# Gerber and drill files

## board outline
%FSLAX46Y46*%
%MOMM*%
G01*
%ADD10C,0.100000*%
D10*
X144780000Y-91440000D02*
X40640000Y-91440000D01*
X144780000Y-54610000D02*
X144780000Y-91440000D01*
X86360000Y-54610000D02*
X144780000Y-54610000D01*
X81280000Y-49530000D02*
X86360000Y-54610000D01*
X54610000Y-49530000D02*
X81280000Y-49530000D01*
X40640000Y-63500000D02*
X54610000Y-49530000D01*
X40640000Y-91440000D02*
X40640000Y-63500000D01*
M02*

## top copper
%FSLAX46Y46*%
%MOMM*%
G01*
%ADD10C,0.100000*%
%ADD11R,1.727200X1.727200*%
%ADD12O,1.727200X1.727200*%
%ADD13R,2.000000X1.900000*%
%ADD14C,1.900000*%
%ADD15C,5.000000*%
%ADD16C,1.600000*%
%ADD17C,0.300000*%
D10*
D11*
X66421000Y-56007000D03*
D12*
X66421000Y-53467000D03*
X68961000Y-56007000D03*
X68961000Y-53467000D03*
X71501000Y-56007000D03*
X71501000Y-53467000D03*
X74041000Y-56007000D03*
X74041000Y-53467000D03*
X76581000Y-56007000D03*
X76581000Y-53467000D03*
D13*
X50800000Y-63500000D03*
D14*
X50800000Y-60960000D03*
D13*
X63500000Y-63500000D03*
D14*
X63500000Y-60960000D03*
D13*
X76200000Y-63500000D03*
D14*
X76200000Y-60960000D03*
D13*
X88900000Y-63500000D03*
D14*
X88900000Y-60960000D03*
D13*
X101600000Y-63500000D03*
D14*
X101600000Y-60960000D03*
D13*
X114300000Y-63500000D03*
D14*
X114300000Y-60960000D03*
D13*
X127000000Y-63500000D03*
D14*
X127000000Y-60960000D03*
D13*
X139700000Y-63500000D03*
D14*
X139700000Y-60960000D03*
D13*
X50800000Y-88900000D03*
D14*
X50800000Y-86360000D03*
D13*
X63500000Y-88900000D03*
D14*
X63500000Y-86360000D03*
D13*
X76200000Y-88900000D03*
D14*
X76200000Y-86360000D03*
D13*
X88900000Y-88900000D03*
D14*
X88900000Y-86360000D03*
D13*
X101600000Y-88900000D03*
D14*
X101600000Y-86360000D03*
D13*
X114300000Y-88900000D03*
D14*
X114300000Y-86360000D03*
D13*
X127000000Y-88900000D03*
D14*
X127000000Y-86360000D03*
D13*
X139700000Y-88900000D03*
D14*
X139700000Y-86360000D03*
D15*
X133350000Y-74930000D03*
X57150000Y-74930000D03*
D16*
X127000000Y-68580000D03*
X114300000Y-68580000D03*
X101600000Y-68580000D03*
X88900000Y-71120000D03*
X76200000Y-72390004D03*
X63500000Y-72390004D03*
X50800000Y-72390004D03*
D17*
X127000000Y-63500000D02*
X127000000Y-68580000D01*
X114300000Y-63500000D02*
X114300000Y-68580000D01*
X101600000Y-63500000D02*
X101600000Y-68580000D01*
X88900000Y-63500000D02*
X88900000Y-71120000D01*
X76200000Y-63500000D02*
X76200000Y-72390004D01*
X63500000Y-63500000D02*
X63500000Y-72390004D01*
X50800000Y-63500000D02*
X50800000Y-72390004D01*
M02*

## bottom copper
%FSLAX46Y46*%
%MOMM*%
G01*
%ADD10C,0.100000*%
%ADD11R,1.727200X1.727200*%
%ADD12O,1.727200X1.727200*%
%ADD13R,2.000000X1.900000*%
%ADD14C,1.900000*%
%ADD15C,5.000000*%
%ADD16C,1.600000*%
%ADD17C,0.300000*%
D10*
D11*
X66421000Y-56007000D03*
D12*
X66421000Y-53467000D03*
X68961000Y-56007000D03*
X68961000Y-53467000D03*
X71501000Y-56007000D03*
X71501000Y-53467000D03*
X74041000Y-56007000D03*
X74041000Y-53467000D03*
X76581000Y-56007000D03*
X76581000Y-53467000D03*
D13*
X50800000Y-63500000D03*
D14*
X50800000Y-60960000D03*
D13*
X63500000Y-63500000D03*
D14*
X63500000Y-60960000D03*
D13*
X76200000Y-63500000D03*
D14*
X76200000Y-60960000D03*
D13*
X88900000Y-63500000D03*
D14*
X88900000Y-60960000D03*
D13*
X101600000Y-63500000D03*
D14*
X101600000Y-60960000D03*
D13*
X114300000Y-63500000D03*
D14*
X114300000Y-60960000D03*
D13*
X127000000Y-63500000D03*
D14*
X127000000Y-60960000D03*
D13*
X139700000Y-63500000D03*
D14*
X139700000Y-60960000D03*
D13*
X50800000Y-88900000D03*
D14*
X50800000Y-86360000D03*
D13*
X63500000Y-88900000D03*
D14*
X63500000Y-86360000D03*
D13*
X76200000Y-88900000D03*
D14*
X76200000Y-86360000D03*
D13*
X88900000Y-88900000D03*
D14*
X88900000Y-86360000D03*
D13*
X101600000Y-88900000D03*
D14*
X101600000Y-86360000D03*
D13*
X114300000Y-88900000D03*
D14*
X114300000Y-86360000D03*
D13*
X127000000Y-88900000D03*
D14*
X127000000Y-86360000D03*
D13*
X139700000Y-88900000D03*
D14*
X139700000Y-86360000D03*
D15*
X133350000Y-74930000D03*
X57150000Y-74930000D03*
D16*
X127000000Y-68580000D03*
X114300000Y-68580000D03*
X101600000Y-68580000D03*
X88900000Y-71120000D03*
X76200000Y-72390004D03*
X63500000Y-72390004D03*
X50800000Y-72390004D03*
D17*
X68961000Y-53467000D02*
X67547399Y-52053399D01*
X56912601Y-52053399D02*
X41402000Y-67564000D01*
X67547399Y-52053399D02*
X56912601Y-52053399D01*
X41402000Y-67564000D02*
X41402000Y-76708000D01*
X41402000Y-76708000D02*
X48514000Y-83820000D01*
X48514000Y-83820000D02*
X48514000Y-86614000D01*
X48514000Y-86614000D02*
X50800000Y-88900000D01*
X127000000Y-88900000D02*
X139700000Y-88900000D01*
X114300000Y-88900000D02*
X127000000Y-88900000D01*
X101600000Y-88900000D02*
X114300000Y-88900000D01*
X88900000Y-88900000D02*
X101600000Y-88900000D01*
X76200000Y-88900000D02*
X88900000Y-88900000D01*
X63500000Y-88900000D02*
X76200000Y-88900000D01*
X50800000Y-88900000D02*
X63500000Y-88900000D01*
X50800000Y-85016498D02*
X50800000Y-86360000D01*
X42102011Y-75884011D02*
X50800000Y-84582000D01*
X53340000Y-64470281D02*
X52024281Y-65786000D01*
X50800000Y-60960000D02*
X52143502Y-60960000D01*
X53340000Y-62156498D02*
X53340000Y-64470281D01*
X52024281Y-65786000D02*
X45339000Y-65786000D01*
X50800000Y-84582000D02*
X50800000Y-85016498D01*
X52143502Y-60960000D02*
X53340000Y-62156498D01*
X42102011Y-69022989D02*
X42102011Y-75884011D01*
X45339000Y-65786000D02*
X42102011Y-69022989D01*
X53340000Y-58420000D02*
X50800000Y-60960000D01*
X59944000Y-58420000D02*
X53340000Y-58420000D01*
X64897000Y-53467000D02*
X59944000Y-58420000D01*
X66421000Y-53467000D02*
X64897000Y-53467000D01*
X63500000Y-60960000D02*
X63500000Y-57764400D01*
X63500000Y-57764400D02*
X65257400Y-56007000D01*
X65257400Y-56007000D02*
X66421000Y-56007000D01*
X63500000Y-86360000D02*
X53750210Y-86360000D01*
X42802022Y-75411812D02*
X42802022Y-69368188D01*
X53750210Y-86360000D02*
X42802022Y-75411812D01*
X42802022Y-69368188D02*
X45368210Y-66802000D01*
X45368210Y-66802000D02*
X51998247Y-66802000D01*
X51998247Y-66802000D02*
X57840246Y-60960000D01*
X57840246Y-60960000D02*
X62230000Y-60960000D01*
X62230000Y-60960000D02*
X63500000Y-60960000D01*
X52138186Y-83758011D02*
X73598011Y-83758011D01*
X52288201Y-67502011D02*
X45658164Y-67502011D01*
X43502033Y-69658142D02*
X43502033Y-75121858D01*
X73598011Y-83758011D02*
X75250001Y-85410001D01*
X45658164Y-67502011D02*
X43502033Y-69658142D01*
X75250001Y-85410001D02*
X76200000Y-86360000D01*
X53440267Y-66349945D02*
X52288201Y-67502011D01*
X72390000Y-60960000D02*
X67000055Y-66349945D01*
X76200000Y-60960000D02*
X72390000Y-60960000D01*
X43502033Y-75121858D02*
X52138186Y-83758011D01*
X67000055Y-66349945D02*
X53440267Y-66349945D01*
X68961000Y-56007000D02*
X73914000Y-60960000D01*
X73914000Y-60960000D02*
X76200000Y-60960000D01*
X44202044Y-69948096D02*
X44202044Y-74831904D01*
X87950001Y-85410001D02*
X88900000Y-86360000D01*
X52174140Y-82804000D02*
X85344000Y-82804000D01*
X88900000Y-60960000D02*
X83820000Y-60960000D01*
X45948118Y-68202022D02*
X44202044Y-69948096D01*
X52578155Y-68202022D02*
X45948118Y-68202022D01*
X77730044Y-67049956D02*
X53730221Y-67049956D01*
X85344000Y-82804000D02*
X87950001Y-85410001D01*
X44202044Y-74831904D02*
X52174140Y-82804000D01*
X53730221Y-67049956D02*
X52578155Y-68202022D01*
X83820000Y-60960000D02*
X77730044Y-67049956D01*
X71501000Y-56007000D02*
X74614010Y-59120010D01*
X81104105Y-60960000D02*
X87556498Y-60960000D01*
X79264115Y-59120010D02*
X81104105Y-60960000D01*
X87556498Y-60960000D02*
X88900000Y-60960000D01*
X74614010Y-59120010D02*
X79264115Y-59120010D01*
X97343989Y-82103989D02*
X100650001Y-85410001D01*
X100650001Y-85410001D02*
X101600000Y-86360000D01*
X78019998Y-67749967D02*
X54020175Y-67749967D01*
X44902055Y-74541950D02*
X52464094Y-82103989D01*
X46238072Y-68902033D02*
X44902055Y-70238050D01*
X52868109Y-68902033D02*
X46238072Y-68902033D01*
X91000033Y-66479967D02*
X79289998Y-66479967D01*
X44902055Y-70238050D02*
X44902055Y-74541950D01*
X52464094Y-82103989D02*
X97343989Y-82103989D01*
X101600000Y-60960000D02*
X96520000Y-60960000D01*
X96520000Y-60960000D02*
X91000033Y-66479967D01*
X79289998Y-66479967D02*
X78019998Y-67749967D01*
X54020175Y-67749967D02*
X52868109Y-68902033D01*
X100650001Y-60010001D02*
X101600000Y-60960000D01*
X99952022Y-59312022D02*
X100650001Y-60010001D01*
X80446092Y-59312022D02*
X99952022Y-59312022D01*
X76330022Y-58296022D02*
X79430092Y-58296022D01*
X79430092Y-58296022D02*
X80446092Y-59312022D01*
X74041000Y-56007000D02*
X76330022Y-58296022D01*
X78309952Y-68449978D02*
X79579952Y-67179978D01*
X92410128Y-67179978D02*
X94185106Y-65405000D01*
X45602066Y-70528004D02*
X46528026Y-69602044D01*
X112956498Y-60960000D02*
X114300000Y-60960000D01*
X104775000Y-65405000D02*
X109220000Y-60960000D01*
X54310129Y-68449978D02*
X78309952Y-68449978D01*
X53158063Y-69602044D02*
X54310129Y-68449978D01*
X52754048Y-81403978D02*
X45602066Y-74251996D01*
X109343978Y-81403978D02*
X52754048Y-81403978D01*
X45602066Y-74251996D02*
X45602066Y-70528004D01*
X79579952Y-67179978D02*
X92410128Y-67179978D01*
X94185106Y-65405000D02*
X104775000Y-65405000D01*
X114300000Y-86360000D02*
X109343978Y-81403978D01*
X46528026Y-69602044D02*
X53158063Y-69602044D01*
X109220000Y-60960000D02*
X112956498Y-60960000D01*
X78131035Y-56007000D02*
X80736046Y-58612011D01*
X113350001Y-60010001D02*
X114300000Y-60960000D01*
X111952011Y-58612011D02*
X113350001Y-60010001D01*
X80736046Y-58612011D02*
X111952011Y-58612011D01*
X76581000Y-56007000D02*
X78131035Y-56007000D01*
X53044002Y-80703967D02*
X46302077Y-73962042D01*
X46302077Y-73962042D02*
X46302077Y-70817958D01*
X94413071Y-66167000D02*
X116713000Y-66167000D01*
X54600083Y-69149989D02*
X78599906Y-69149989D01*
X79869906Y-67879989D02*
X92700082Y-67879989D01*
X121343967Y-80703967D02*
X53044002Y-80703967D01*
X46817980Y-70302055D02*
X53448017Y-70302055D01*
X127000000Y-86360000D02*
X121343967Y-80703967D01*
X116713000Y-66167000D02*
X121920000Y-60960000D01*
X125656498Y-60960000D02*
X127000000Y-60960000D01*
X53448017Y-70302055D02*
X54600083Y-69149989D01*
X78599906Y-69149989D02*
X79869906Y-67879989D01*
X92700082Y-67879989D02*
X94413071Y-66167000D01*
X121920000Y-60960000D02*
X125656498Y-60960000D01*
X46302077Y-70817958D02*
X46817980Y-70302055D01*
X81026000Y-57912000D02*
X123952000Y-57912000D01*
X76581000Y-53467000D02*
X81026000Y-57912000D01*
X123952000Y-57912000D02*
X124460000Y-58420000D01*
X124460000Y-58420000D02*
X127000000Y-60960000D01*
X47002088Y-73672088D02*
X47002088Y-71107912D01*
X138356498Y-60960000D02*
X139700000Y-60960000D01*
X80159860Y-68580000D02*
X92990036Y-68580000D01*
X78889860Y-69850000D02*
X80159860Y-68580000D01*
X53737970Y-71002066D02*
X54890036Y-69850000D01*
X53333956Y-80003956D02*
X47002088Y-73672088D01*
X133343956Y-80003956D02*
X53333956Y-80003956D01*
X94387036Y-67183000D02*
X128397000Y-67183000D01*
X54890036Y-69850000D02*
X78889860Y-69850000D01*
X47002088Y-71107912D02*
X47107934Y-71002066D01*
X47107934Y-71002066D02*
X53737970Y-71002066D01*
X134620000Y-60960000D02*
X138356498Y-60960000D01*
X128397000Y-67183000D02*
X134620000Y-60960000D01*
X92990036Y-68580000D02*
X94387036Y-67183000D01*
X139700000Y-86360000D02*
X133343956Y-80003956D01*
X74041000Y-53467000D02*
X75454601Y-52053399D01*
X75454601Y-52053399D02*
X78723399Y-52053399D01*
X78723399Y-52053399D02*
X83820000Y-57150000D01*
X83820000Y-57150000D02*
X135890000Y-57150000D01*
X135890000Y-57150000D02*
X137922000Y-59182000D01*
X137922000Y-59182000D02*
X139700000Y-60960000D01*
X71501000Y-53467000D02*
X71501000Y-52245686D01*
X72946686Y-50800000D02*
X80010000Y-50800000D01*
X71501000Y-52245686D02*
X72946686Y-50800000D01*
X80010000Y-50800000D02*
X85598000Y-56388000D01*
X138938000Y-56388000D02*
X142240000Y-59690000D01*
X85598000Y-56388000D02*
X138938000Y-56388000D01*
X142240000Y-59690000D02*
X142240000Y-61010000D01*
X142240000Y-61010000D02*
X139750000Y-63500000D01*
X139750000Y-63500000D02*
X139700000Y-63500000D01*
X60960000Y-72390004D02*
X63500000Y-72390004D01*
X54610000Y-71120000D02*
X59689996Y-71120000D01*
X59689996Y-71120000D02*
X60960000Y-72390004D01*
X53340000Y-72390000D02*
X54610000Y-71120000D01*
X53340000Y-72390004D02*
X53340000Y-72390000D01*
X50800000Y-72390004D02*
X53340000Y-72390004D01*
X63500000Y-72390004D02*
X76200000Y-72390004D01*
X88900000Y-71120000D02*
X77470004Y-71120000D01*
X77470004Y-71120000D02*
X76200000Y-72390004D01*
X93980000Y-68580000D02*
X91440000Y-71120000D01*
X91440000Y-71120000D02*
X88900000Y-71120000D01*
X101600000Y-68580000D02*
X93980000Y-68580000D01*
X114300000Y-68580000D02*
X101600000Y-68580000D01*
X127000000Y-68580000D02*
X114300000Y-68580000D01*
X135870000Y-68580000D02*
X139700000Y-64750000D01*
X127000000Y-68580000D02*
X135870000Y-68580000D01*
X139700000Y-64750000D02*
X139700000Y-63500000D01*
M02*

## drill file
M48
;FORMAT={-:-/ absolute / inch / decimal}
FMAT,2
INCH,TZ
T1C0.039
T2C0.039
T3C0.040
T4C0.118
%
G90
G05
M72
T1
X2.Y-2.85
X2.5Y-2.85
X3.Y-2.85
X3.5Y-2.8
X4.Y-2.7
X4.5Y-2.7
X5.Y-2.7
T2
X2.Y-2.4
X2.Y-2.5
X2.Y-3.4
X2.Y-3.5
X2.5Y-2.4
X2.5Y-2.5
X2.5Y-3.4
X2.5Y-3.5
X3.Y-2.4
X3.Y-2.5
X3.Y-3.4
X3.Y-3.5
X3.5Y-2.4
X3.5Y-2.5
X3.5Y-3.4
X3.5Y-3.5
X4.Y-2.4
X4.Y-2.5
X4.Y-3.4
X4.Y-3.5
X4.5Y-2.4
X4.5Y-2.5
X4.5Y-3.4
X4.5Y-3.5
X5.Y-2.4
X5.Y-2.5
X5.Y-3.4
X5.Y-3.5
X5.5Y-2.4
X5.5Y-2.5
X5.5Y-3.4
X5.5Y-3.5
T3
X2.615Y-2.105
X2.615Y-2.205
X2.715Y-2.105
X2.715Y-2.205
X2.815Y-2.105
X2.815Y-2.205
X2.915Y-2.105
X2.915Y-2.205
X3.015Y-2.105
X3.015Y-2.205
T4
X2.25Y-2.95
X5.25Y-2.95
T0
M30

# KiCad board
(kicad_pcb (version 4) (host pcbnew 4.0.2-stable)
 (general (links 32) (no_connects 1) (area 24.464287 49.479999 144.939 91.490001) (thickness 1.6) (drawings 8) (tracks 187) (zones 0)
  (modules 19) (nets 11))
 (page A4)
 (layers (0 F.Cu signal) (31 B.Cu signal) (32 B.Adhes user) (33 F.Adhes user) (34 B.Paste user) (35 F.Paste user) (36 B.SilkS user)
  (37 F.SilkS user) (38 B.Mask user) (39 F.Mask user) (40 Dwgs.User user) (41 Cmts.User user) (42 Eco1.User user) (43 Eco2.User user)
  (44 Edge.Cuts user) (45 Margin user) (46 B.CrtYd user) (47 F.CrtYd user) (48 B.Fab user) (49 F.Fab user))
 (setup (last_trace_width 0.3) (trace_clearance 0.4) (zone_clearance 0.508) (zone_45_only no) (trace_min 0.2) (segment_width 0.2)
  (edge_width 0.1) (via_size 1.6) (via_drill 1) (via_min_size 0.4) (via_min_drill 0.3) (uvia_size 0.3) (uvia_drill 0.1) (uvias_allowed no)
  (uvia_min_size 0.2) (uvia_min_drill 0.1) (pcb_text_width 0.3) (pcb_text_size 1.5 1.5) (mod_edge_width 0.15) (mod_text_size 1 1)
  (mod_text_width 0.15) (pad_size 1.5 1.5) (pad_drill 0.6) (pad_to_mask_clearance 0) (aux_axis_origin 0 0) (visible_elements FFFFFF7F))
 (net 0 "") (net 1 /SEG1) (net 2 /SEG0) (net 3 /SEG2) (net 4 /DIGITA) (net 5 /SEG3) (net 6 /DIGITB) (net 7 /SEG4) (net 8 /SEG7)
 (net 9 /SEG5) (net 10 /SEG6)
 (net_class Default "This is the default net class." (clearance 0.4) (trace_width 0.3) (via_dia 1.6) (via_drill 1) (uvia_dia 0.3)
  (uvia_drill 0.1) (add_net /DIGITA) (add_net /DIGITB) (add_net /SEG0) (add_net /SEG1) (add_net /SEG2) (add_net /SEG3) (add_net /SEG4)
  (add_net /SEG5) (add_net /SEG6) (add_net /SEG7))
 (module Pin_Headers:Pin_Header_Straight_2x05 (layer F.Cu) (at 66.421 56.007 90)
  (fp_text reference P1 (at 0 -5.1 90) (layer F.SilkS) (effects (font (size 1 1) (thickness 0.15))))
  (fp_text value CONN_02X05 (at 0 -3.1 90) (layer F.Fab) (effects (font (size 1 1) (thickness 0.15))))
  (pad 1 thru_hole rect (at 0 0 90) (size 1.7272 1.7272) (drill 1.016) (layers *.Cu *.Mask F.SilkS) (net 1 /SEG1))
  (pad 2 thru_hole oval (at 2.54 0 90) (size 1.7272 1.7272) (drill 1.016) (layers *.Cu *.Mask F.SilkS) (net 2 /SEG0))
  (pad 3 thru_hole oval (at 0 2.54 90) (size 1.7272 1.7272) (drill 1.016) (layers *.Cu *.Mask F.SilkS) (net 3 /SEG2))
  (pad 4 thru_hole oval (at 2.54 2.54 90) (size 1.7272 1.7272) (drill 1.016) (layers *.Cu *.Mask F.SilkS) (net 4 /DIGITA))
  (pad 5 thru_hole oval (at 0 5.08 90) (size 1.7272 1.7272) (drill 1.016) (layers *.Cu *.Mask F.SilkS) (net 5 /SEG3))
  (pad 6 thru_hole oval (at 2.54 5.08 90) (size 1.7272 1.7272) (drill 1.016) (layers *.Cu *.Mask F.SilkS) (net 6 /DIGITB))
  (pad 7 thru_hole oval (at 0 7.62 90) (size 1.7272 1.7272) (drill 1.016) (layers *.Cu *.Mask F.SilkS) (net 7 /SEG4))
  (pad 8 thru_hole oval (at 2.54 7.62 90) (size 1.7272 1.7272) (drill 1.016) (layers *.Cu *.Mask F.SilkS) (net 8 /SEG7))
  (pad 9 thru_hole oval (at 0 10.16 90) (size 1.7272 1.7272) (drill 1.016) (layers *.Cu *.Mask F.SilkS) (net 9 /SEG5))
  (pad 10 thru_hole oval (at 2.54 10.16 90) (size 1.7272 1.7272) (drill 1.016) (layers *.Cu *.Mask F.SilkS) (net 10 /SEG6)))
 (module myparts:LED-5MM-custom (layer F.Cu) (at 50.8 63.5 90)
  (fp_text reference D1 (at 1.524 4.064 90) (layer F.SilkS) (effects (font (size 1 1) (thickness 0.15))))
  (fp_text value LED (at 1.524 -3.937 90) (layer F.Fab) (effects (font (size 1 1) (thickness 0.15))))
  (pad 1 thru_hole rect (at 0 0 180) (size 2 1.9) (drill 1.00076) (layers *.Cu *.Mask F.SilkS) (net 6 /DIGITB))
  (pad 2 thru_hole circle (at 2.54 0 90) (size 1.9 1.9) (drill 1.00076) (layers *.Cu *.Mask F.SilkS) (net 2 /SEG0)))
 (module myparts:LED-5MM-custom (layer F.Cu) (at 63.5 63.5 90)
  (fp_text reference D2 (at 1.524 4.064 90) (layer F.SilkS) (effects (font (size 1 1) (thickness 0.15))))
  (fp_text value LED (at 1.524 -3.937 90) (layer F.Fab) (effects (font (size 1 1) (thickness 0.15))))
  (pad 1 thru_hole rect (at 0 0 180) (size 2 1.9) (drill 1.00076) (layers *.Cu *.Mask F.SilkS) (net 6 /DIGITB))
  (pad 2 thru_hole circle (at 2.54 0 90) (size 1.9 1.9) (drill 1.00076) (layers *.Cu *.Mask F.SilkS) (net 1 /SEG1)))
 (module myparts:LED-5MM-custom (layer F.Cu) (at 76.2 63.5 90)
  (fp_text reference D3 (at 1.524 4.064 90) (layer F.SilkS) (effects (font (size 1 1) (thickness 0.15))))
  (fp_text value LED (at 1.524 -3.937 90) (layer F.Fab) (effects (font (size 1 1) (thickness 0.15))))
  (pad 1 thru_hole rect (at 0 0 180) (size 2 1.9) (drill 1.00076) (layers *.Cu *.Mask F.SilkS) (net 6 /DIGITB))
  (pad 2 thru_hole circle (at 2.54 0 90) (size 1.9 1.9) (drill 1.00076) (layers *.Cu *.Mask F.SilkS) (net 3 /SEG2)))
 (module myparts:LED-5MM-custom (layer F.Cu) (at 88.9 63.5 90)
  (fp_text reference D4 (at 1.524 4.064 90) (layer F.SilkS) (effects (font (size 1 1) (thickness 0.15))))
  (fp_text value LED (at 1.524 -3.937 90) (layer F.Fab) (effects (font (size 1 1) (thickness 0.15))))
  (pad 1 thru_hole rect (at 0 0 180) (size 2 1.9) (drill 1.00076) (layers *.Cu *.Mask F.SilkS) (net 6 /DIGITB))
  (pad 2 thru_hole circle (at 2.54 0 90) (size 1.9 1.9) (drill 1.00076) (layers *.Cu *.Mask F.SilkS) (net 5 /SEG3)))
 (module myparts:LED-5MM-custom (layer F.Cu) (at 101.6 63.5 90)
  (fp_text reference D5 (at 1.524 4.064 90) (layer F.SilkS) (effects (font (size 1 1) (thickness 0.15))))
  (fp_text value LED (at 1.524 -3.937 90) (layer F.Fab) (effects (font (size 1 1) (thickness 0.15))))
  (pad 1 thru_hole rect (at 0 0 180) (size 2 1.9) (drill 1.00076) (layers *.Cu *.Mask F.SilkS) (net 6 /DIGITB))
  (pad 2 thru_hole circle (at 2.54 0 90) (size 1.9 1.9) (drill 1.00076) (layers *.Cu *.Mask F.SilkS) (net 7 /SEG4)))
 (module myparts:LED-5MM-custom (layer F.Cu) (at 114.3 63.5 90)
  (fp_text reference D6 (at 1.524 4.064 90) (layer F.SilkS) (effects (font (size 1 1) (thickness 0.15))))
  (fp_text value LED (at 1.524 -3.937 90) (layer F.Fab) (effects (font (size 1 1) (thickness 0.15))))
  (pad 1 thru_hole rect (at 0 0 180) (size 2 1.9) (drill 1.00076) (layers *.Cu *.Mask F.SilkS) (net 6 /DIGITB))
  (pad 2 thru_hole circle (at 2.54 0 90) (size 1.9 1.9) (drill 1.00076) (layers *.Cu *.Mask F.SilkS) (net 9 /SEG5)))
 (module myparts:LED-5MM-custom (layer F.Cu) (at 127 63.5 90)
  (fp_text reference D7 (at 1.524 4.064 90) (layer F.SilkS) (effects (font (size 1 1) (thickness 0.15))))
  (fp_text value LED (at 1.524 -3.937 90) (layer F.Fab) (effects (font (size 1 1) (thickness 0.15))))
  (pad 1 thru_hole rect (at 0 0 180) (size 2 1.9) (drill 1.00076) (layers *.Cu *.Mask F.SilkS) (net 6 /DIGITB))
  (pad 2 thru_hole circle (at 2.54 0 90) (size 1.9 1.9) (drill 1.00076) (layers *.Cu *.Mask F.SilkS) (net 10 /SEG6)))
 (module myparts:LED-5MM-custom (layer F.Cu) (at 139.7 63.5 90)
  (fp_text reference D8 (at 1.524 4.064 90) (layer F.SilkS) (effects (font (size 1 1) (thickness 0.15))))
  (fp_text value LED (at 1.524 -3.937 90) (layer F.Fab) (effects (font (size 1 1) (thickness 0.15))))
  (pad 1 thru_hole rect (at 0 0 180) (size 2 1.9) (drill 1.00076) (layers *.Cu *.Mask F.SilkS) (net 6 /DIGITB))
  (pad 2 thru_hole circle (at 2.54 0 90) (size 1.9 1.9) (drill 1.00076) (layers *.Cu *.Mask F.SilkS) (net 8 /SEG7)))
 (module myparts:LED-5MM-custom (layer F.Cu) (at 50.8 88.9 90)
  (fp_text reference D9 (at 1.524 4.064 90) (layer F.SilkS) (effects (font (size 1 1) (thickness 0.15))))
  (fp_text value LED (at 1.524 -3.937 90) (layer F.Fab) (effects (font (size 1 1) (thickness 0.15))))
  (pad 1 thru_hole rect (at 0 0 180) (size 2 1.9) (drill 1.00076) (layers *.Cu *.Mask F.SilkS) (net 4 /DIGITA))
  (pad 2 thru_hole circle (at 2.54 0 90) (size 1.9 1.9) (drill 1.00076) (layers *.Cu *.Mask F.SilkS) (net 2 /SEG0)))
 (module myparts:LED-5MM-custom (layer F.Cu) (at 63.5 88.9 90)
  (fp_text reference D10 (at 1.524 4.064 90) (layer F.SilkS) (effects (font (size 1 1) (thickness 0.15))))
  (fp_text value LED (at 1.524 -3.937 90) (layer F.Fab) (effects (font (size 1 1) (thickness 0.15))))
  (pad 1 thru_hole rect (at 0 0 180) (size 2 1.9) (drill 1.00076) (layers *.Cu *.Mask F.SilkS) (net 4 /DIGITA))
  (pad 2 thru_hole circle (at 2.54 0 90) (size 1.9 1.9) (drill 1.00076) (layers *.Cu *.Mask F.SilkS) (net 1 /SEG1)))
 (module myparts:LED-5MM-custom (layer F.Cu) (at 76.2 88.9 90)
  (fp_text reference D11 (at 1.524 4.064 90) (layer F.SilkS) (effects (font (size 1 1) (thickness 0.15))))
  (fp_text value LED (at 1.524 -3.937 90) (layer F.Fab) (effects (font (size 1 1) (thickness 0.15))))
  (pad 1 thru_hole rect (at 0 0 180) (size 2 1.9) (drill 1.00076) (layers *.Cu *.Mask F.SilkS) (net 4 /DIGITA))
  (pad 2 thru_hole circle (at 2.54 0 90) (size 1.9 1.9) (drill 1.00076) (layers *.Cu *.Mask F.SilkS) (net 3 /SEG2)))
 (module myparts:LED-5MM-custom (layer F.Cu) (at 88.9 88.9 90)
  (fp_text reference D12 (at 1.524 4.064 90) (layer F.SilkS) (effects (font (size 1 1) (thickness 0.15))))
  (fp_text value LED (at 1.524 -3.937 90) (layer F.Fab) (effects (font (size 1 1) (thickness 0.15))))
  (pad 1 thru_hole rect (at 0 0 180) (size 2 1.9) (drill 1.00076) (layers *.Cu *.Mask F.SilkS) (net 4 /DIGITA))
  (pad 2 thru_hole circle (at 2.54 0 90) (size 1.9 1.9) (drill 1.00076) (layers *.Cu *.Mask F.SilkS) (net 5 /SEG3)))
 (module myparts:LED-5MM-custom (layer F.Cu) (at 101.6 88.9 90)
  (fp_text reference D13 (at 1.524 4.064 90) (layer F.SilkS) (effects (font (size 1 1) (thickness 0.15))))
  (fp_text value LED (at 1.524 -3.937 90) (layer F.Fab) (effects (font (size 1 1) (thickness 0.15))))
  (pad 1 thru_hole rect (at 0 0 180) (size 2 1.9) (drill 1.00076) (layers *.Cu *.Mask F.SilkS) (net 4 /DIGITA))
  (pad 2 thru_hole circle (at 2.54 0 90) (size 1.9 1.9) (drill 1.00076) (layers *.Cu *.Mask F.SilkS) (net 7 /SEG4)))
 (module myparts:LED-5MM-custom (layer F.Cu) (at 114.3 88.9 90)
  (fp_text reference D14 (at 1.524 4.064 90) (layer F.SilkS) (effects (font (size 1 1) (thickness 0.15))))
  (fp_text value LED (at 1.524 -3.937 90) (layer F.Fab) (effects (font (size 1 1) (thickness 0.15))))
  (pad 1 thru_hole rect (at 0 0 180) (size 2 1.9) (drill 1.00076) (layers *.Cu *.Mask F.SilkS) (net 4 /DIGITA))
  (pad 2 thru_hole circle (at 2.54 0 90) (size 1.9 1.9) (drill 1.00076) (layers *.Cu *.Mask F.SilkS) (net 9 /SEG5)))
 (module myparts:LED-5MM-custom (layer F.Cu) (at 127 88.9 90)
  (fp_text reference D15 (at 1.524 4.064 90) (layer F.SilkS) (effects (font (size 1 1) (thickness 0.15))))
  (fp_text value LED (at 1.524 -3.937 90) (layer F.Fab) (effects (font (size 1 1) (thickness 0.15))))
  (pad 1 thru_hole rect (at 0 0 180) (size 2 1.9) (drill 1.00076) (layers *.Cu *.Mask F.SilkS) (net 4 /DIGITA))
  (pad 2 thru_hole circle (at 2.54 0 90) (size 1.9 1.9) (drill 1.00076) (layers *.Cu *.Mask F.SilkS) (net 10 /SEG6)))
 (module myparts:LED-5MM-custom (layer F.Cu) (at 139.7 88.9 90)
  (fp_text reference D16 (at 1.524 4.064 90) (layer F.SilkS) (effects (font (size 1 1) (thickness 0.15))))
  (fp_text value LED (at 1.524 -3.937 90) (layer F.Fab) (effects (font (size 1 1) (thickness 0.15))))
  (pad 1 thru_hole rect (at 0 0 180) (size 2 1.9) (drill 1.00076) (layers *.Cu *.Mask F.SilkS) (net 4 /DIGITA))
  (pad 2 thru_hole circle (at 2.54 0 90) (size 1.9 1.9) (drill 1.00076) (layers *.Cu *.Mask F.SilkS) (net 8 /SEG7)))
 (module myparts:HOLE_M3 (layer F.Cu) (at 133.35 74.93)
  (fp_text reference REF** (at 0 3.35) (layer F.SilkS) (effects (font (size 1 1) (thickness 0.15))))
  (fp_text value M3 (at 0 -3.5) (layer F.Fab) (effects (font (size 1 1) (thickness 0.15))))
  (pad 1 thru_hole circle (at 0 0) (size 5 5) (drill 3) (layers *.Cu *.Mask F.SilkS)))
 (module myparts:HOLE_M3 (layer F.Cu) (at 57.15 74.93)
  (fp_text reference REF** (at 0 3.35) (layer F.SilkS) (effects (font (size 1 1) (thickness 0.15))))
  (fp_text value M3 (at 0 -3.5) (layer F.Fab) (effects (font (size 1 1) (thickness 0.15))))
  (pad 1 thru_hole circle (at 0 0) (size 5 5) (drill 3) (layers *.Cu *.Mask F.SilkS)))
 (gr_line (start 144.78 91.44) (end 40.64 91.44) (layer Edge.Cuts) (width 0.1))
 (gr_line (start 144.78 54.61) (end 144.78 91.44) (layer Edge.Cuts) (width 0.1))
 (gr_line (start 86.36 54.61) (end 144.78 54.61) (layer Edge.Cuts) (width 0.1))
 (gr_line (start 81.28 49.53) (end 86.36 54.61) (layer Edge.Cuts) (width 0.1))
 (gr_line (start 54.61 49.53) (end 81.28 49.53) (layer Edge.Cuts) (width 0.1))
 (gr_line (start 40.64 63.5) (end 54.61 49.53) (layer Edge.Cuts) (width 0.1))
 (gr_line (start 40.64 91.44) (end 40.64 63.5) (layer Edge.Cuts) (width 0.1))
 (segment (start 68.961 53.467) (end 67.547399 52.053399) (width 0.3) (layer B.Cu) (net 4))
 (segment (start 56.912601 52.053399) (end 41.402 67.564) (width 0.3) (layer B.Cu) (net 4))
 (segment (start 67.547399 52.053399) (end 56.912601 52.053399) (width 0.3) (layer B.Cu) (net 4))
 (segment (start 41.402 67.564) (end 41.402 76.708) (width 0.3) (layer B.Cu) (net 4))
 (segment (start 41.402 76.708) (end 48.514 83.82) (width 0.3) (layer B.Cu) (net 4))
 (segment (start 48.514 83.82) (end 48.514 86.614) (width 0.3) (layer B.Cu) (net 4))
 (segment (start 48.514 86.614) (end 50.8 88.9) (width 0.3) (layer B.Cu) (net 4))
 (segment (start 127 88.9) (end 139.7 88.9) (width 0.3) (layer B.Cu) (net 4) (status 30))
 (segment (start 114.3 88.9) (end 127 88.9) (width 0.3) (layer B.Cu) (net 4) (status 30))
 (segment (start 101.6 88.9) (end 114.3 88.9) (width 0.3) (layer B.Cu) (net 4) (status 30))
 (segment (start 88.9 88.9) (end 101.6 88.9) (width 0.3) (layer B.Cu) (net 4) (status 30))
 (segment (start 76.2 88.9) (end 88.9 88.9) (width 0.3) (layer B.Cu) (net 4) (status 30))
 (segment (start 63.5 88.9) (end 76.2 88.9) (width 0.3) (layer B.Cu) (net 4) (status 30))
 (segment (start 50.8 88.9) (end 63.5 88.9) (width 0.3) (layer B.Cu) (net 4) (status 30))
 (segment (start 50.8 85.016498) (end 50.8 86.36) (width 0.3) (layer B.Cu) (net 2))
 (segment (start 42.102011 75.884011) (end 50.8 84.582) (width 0.3) (layer B.Cu) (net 2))
 (segment (start 53.34 64.470281) (end 52.024281 65.786) (width 0.3) (layer B.Cu) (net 2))
 (segment (start 50.8 60.96) (end 52.143502 60.96) (width 0.3) (layer B.Cu) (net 2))
 (segment (start 53.34 62.156498) (end 53.34 64.470281) (width 0.3) (layer B.Cu) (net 2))
 (segment (start 52.024281 65.786) (end 45.339 65.786) (width 0.3) (layer B.Cu) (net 2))
 (segment (start 50.8 84.582) (end 50.8 85.016498) (width 0.3) (layer B.Cu) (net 2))
 (segment (start 52.143502 60.96) (end 53.34 62.156498) (width 0.3) (layer B.Cu) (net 2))
 (segment (start 42.102011 69.022989) (end 42.102011 75.884011) (width 0.3) (layer B.Cu) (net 2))
 (segment (start 45.339 65.786) (end 42.102011 69.022989) (width 0.3) (layer B.Cu) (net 2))
 (segment (start 53.34 58.42) (end 50.8 60.96) (width 0.3) (layer B.Cu) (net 2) (status 20))
 (segment (start 59.944 58.42) (end 53.34 58.42) (width 0.3) (layer B.Cu) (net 2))
 (segment (start 64.897 53.467) (end 59.944 58.42) (width 0.3) (layer B.Cu) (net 2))
 (segment (start 66.421 53.467) (end 64.897 53.467) (width 0.3) (layer B.Cu) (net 2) (status 10))
 (segment (start 63.5 60.96) (end 63.5 57.7644) (width 0.3) (layer B.Cu) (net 1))
 (segment (start 63.5 57.7644) (end 65.2574 56.007) (width 0.3) (layer B.Cu) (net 1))
 (segment (start 65.2574 56.007) (end 66.421 56.007) (width 0.3) (layer B.Cu) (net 1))
 (segment (start 63.5 86.36) (end 53.75021 86.36) (width 0.3) (layer B.Cu) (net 1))
 (segment (start 42.802022 75.411812) (end 42.802022 69.368188) (width 0.3) (layer B.Cu) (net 1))
 (segment (start 53.75021 86.36) (end 42.802022 75.411812) (width 0.3) (layer B.Cu) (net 1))
 (segment (start 42.802022 69.368188) (end 45.36821 66.802) (width 0.3) (layer B.Cu) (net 1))
 (segment (start 45.36821 66.802) (end 51.998247 66.802) (width 0.3) (layer B.Cu) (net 1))
 (segment (start 51.998247 66.802) (end 57.840246 60.96) (width 0.3) (layer B.Cu) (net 1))
 (segment (start 57.840246 60.96) (end 62.23 60.96) (width 0.3) (layer B.Cu) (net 1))
 (segment (start 62.23 60.96) (end 63.5 60.96) (width 0.3) (layer B.Cu) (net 1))
 (segment (start 52.138186 83.758011) (end 73.598011 83.758011) (width 0.3) (layer B.Cu) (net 3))
 (segment (start 52.288201 67.502011) (end 45.658164 67.502011) (width 0.3) (layer B.Cu) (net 3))
 (segment (start 43.502033 69.658142) (end 43.502033 75.121858) (width 0.3) (layer B.Cu) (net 3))
 (segment (start 73.598011 83.758011) (end 75.250001 85.410001) (width 0.3) (layer B.Cu) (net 3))
 (segment (start 45.658164 67.502011) (end 43.502033 69.658142) (width 0.3) (layer B.Cu) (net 3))
 (segment (start 75.250001 85.410001) (end 76.2 86.36) (width 0.3) (layer B.Cu) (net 3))
 (segment (start 53.440267 66.349945) (end 52.288201 67.502011) (width 0.3) (layer B.Cu) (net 3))
 (segment (start 72.39 60.96) (end 67.000055 66.349945) (width 0.3) (layer B.Cu) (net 3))
 (segment (start 76.2 60.96) (end 72.39 60.96) (width 0.3) (layer B.Cu) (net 3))
 (segment (start 43.502033 75.121858) (end 52.138186 83.758011) (width 0.3) (layer B.Cu) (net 3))
 (segment (start 67.000055 66.349945) (end 53.440267 66.349945) (width 0.3) (layer B.Cu) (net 3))
 (segment (start 68.961 56.007) (end 73.914 60.96) (width 0.3) (layer B.Cu) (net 3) (status 10))
 (segment (start 73.914 60.96) (end 76.2 60.96) (width 0.3) (layer B.Cu) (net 3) (status 20))
 (segment (start 44.202044 69.948096) (end 44.202044 74.831904) (width 0.3) (layer B.Cu) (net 5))
 (segment (start 87.950001 85.410001) (end 88.9 86.36) (width 0.3) (layer B.Cu) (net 5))
 (segment (start 52.17414 82.804) (end 85.344 82.804) (width 0.3) (layer B.Cu) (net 5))
 (segment (start 88.9 60.96) (end 83.82 60.96) (width 0.3) (layer B.Cu) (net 5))
 (segment (start 45.948118 68.202022) (end 44.202044 69.948096) (width 0.3) (layer B.Cu) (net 5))
 (segment (start 52.578155 68.202022) (end 45.948118 68.202022) (width 0.3) (layer B.Cu) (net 5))
 (segment (start 77.730044 67.049956) (end 53.730221 67.049956) (width 0.3) (layer B.Cu) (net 5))
 (segment (start 85.344 82.804) (end 87.950001 85.410001) (width 0.3) (layer B.Cu) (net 5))
 (segment (start 44.202044 74.831904) (end 52.17414 82.804) (width 0.3) (layer B.Cu) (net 5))
 (segment (start 53.730221 67.049956) (end 52.578155 68.202022) (width 0.3) (layer B.Cu) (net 5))
 (segment (start 83.82 60.96) (end 77.730044 67.049956) (width 0.3) (layer B.Cu) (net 5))
 (segment (start 71.501 56.007) (end 74.61401 59.12001) (width 0.3) (layer B.Cu) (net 5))
 (segment (start 81.104105 60.96) (end 87.556498 60.96) (width 0.3) (layer B.Cu) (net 5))
 (segment (start 79.264115 59.12001) (end 81.104105 60.96) (width 0.3) (layer B.Cu) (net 5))
 (segment (start 87.556498 60.96) (end 88.9 60.96) (width 0.3) (layer B.Cu) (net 5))
 (segment (start 74.61401 59.12001) (end 79.264115 59.12001) (width 0.3) (layer B.Cu) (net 5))
 (segment (start 97.343989 82.103989) (end 100.650001 85.410001) (width 0.3) (layer B.Cu) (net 7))
 (segment (start 100.650001 85.410001) (end 101.6 86.36) (width 0.3) (layer B.Cu) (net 7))
 (segment (start 78.019998 67.749967) (end 54.020175 67.749967) (width 0.3) (layer B.Cu) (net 7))
 (segment (start 44.902055 74.54195) (end 52.464094 82.103989) (width 0.3) (layer B.Cu) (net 7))
 (segment (start 46.238072 68.902033) (end 44.902055 70.23805) (width 0.3) (layer B.Cu) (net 7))
 (segment (start 52.868109 68.902033) (end 46.238072 68.902033) (width 0.3) (layer B.Cu) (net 7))
 (segment (start 91.000033 66.479967) (end 79.289998 66.479967) (width 0.3) (layer B.Cu) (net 7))
 (segment (start 44.902055 70.23805) (end 44.902055 74.54195) (width 0.3) (layer B.Cu) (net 7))
 (segment (start 52.464094 82.103989) (end 97.343989 82.103989) (width 0.3) (layer B.Cu) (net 7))
 (segment (start 101.6 60.96) (end 96.52 60.96) (width 0.3) (layer B.Cu) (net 7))
 (segment (start 96.52 60.96) (end 91.000033 66.479967) (width 0.3) (layer B.Cu) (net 7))
 (segment (start 79.289998 66.479967) (end 78.019998 67.749967) (width 0.3) (layer B.Cu) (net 7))
 (segment (start 54.020175 67.749967) (end 52.868109 68.902033) (width 0.3) (layer B.Cu) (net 7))
 (segment (start 100.650001 60.010001) (end 101.6 60.96) (width 0.3) (layer B.Cu) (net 7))
 (segment (start 99.952022 59.312022) (end 100.650001 60.010001) (width 0.3) (layer B.Cu) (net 7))
 (segment (start 80.446092 59.312022) (end 99.952022 59.312022) (width 0.3) (layer B.Cu) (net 7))
 (segment (start 76.330022 58.296022) (end 79.430092 58.296022) (width 0.3) (layer B.Cu) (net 7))
 (segment (start 79.430092 58.296022) (end 80.446092 59.312022) (width 0.3) (layer B.Cu) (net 7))
 (segment (start 74.041 56.007) (end 76.330022 58.296022) (width 0.3) (layer B.Cu) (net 7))
 (segment (start 78.309952 68.449978) (end 79.579952 67.179978) (width 0.3) (layer B.Cu) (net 9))
 (segment (start 92.410128 67.179978) (end 94.185106 65.405) (width 0.3) (layer B.Cu) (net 9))
 (segment (start 45.602066 70.528004) (end 46.528026 69.602044) (width 0.3) (layer B.Cu) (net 9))
 (segment (start 112.956498 60.96) (end 114.3 60.96) (width 0.3) (layer B.Cu) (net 9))
 (segment (start 104.775 65.405) (end 109.22 60.96) (width 0.3) (layer B.Cu) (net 9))
 (segment (start 54.310129 68.449978) (end 78.309952 68.449978) (width 0.3) (layer B.Cu) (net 9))
 (segment (start 53.158063 69.602044) (end 54.310129 68.449978) (width 0.3) (layer B.Cu) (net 9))
 (segment (start 52.754048 81.403978) (end 45.602066 74.251996) (width 0.3) (layer B.Cu) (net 9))
 (segment (start 109.343978 81.403978) (end 52.754048 81.403978) (width 0.3) (layer B.Cu) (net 9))
 (segment (start 45.602066 74.251996) (end 45.602066 70.528004) (width 0.3) (layer B.Cu) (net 9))
 (segment (start 79.579952 67.179978) (end 92.410128 67.179978) (width 0.3) (layer B.Cu) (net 9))
 (segment (start 94.185106 65.405) (end 104.775 65.405) (width 0.3) (layer B.Cu) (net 9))
 (segment (start 114.3 86.36) (end 109.343978 81.403978) (width 0.3) (layer B.Cu) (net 9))
 (segment (start 46.528026 69.602044) (end 53.158063 69.602044) (width 0.3) (layer B.Cu) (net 9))
 (segment (start 109.22 60.96) (end 112.956498 60.96) (width 0.3) (layer B.Cu) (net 9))
 (segment (start 78.131035 56.007) (end 80.736046 58.612011) (width 0.3) (layer B.Cu) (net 9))
 (segment (start 113.350001 60.010001) (end 114.3 60.96) (width 0.3) (layer B.Cu) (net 9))
 (segment (start 111.952011 58.612011) (end 113.350001 60.010001) (width 0.3) (layer B.Cu) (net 9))
 (segment (start 80.736046 58.612011) (end 111.952011 58.612011) (width 0.3) (layer B.Cu) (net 9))
 (segment (start 76.581 56.007) (end 78.131035 56.007) (width 0.3) (layer B.Cu) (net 9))
 (segment (start 53.044002 80.703967) (end 46.302077 73.962042) (width 0.3) (layer B.Cu) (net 10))
 (segment (start 46.302077 73.962042) (end 46.302077 70.817958) (width 0.3) (layer B.Cu) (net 10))
 (segment (start 94.413071 66.167) (end 116.713 66.167) (width 0.3) (layer B.Cu) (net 10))
 (segment (start 54.600083 69.149989) (end 78.599906 69.149989) (width 0.3) (layer B.Cu) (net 10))
 (segment (start 79.869906 67.879989) (end 92.700082 67.879989) (width 0.3) (layer B.Cu) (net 10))
 (segment (start 121.343967 80.703967) (end 53.044002 80.703967) (width 0.3) (layer B.Cu) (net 10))
 (segment (start 46.81798 70.302055) (end 53.448017 70.302055) (width 0.3) (layer B.Cu) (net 10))
 (segment (start 127 86.36) (end 121.343967 80.703967) (width 0.3) (layer B.Cu) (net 10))
 (segment (start 116.713 66.167) (end 121.92 60.96) (width 0.3) (layer B.Cu) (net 10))
 (segment (start 125.656498 60.96) (end 127 60.96) (width 0.3) (layer B.Cu) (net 10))
 (segment (start 53.448017 70.302055) (end 54.600083 69.149989) (width 0.3) (layer B.Cu) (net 10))
 (segment (start 78.599906 69.149989) (end 79.869906 67.879989) (width 0.3) (layer B.Cu) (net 10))
 (segment (start 92.700082 67.879989) (end 94.413071 66.167) (width 0.3) (layer B.Cu) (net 10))
 (segment (start 121.92 60.96) (end 125.656498 60.96) (width 0.3) (layer B.Cu) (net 10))
 (segment (start 46.302077 70.817958) (end 46.81798 70.302055) (width 0.3) (layer B.Cu) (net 10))
 (segment (start 81.026 57.912) (end 123.952 57.912) (width 0.3) (layer B.Cu) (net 10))
 (segment (start 76.581 53.467) (end 81.026 57.912) (width 0.3) (layer B.Cu) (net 10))
 (segment (start 123.952 57.912) (end 124.46 58.42) (width 0.3) (layer B.Cu) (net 10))
 (segment (start 124.46 58.42) (end 127 60.96) (width 0.3) (layer B.Cu) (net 10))
 (segment (start 47.002088 73.672088) (end 47.002088 71.107912) (width 0.3) (layer B.Cu) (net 8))
 (segment (start 138.356498 60.96) (end 139.7 60.96) (width 0.3) (layer B.Cu) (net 8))
 (segment (start 80.15986 68.58) (end 92.990036 68.58) (width 0.3) (layer B.Cu) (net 8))
 (segment (start 78.88986 69.85) (end 80.15986 68.58) (width 0.3) (layer B.Cu) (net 8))
 (segment (start 53.73797 71.002066) (end 54.890036 69.85) (width 0.3) (layer B.Cu) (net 8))
 (segment (start 53.333956 80.003956) (end 47.002088 73.672088) (width 0.3) (layer B.Cu) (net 8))
 (segment (start 133.343956 80.003956) (end 53.333956 80.003956) (width 0.3) (layer B.Cu) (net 8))
 (segment (start 94.387036 67.183) (end 128.397 67.183) (width 0.3) (layer B.Cu) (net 8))
 (segment (start 54.890036 69.85) (end 78.88986 69.85) (width 0.3) (layer B.Cu) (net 8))
 (segment (start 47.002088 71.107912) (end 47.107934 71.002066) (width 0.3) (layer B.Cu) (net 8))
 (segment (start 47.107934 71.002066) (end 53.73797 71.002066) (width 0.3) (layer B.Cu) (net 8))
 (segment (start 134.62 60.96) (end 138.356498 60.96) (width 0.3) (layer B.Cu) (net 8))
 (segment (start 128.397 67.183) (end 134.62 60.96) (width 0.3) (layer B.Cu) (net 8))
 (segment (start 92.990036 68.58) (end 94.387036 67.183) (width 0.3) (layer B.Cu) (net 8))
 (segment (start 139.7 86.36) (end 133.343956 80.003956) (width 0.3) (layer B.Cu) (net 8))
 (segment (start 74.041 53.467) (end 75.454601 52.053399) (width 0.3) (layer B.Cu) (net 8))
 (segment (start 75.454601 52.053399) (end 78.723399 52.053399) (width 0.3) (layer B.Cu) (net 8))
 (segment (start 78.723399 52.053399) (end 83.82 57.15) (width 0.3) (layer B.Cu) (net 8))
 (segment (start 83.82 57.15) (end 135.89 57.15) (width 0.3) (layer B.Cu) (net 8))
 (segment (start 135.89 57.15) (end 137.922 59.182) (width 0.3) (layer B.Cu) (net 8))
 (segment (start 137.922 59.182) (end 139.7 60.96) (width 0.3) (layer B.Cu) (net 8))
 (segment (start 71.501 53.467) (end 71.501 52.245686) (width 0.3) (layer B.Cu) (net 6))
 (segment (start 72.946686 50.8) (end 80.01 50.8) (width 0.3) (layer B.Cu) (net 6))
 (segment (start 71.501 52.245686) (end 72.946686 50.8) (width 0.3) (layer B.Cu) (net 6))
 (segment (start 80.01 50.8) (end 85.598 56.388) (width 0.3) (layer B.Cu) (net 6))
 (segment (start 138.938 56.388) (end 142.24 59.69) (width 0.3) (layer B.Cu) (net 6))
 (segment (start 85.598 56.388) (end 138.938 56.388) (width 0.3) (layer B.Cu) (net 6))
 (segment (start 142.24 59.69) (end 142.24 61.01) (width 0.3) (layer B.Cu) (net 6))
 (segment (start 142.24 61.01) (end 139.75 63.5) (width 0.3) (layer B.Cu) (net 6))
 (segment (start 139.75 63.5) (end 139.7 63.5) (width 0.3) (layer B.Cu) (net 6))
 (segment (start 60.96 72.390004) (end 63.5 72.390004) (width 0.3) (layer B.Cu) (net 6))
 (segment (start 54.61 71.12) (end 59.689996 71.12) (width 0.3) (layer B.Cu) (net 6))
 (segment (start 59.689996 71.12) (end 60.96 72.390004) (width 0.3) (layer B.Cu) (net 6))
 (segment (start 53.34 72.39) (end 54.61 71.12) (width 0.3) (layer B.Cu) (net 6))
 (segment (start 53.34 72.390004) (end 53.34 72.39) (width 0.3) (layer B.Cu) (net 6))
 (segment (start 50.8 72.390004) (end 53.34 72.390004) (width 0.3) (layer B.Cu) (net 6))
 (segment (start 63.5 72.390004) (end 76.2 72.390004) (width 0.3) (layer B.Cu) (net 6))
 (segment (start 88.9 71.12) (end 77.470004 71.12) (width 0.3) (layer B.Cu) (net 6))
 (segment (start 77.470004 71.12) (end 76.2 72.390004) (width 0.3) (layer B.Cu) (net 6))
 (segment (start 93.98 68.58) (end 91.44 71.12) (width 0.3) (layer B.Cu) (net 6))
 (segment (start 91.44 71.12) (end 88.9 71.12) (width 0.3) (layer B.Cu) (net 6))
 (segment (start 101.6 68.58) (end 93.98 68.58) (width 0.3) (layer B.Cu) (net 6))
 (segment (start 114.3 68.58) (end 101.6 68.58) (width 0.3) (layer B.Cu) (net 6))
 (segment (start 127 68.58) (end 114.3 68.58) (width 0.3) (layer B.Cu) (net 6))
 (segment (start 135.87 68.58) (end 139.7 64.75) (width 0.3) (layer B.Cu) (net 6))
 (segment (start 127 68.58) (end 135.87 68.58) (width 0.3) (layer B.Cu) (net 6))
 (segment (start 127 63.5) (end 127 68.58) (width 0.3) (layer F.Cu) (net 6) (status 10))
 (via (at 127 68.58) (size 1.6) (drill 1) (layers F.Cu B.Cu) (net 6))
 (segment (start 114.3 63.5) (end 114.3 68.58) (width 0.3) (layer F.Cu) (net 6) (status 10))
 (via (at 114.3 68.58) (size 1.6) (drill 1) (layers F.Cu B.Cu) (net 6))
 (segment (start 101.6 63.5) (end 101.6 68.58) (width 0.3) (layer F.Cu) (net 6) (status 10))
 (via (at 101.6 68.58) (size 1.6) (drill 1) (layers F.Cu B.Cu) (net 6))
 (segment (start 88.9 63.5) (end 88.9 71.12) (width 0.3) (layer F.Cu) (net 6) (status 10))
 (via (at 88.9 71.12) (size 1.6) (drill 1) (layers F.Cu B.Cu) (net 6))
 (segment (start 76.2 63.5) (end 76.2 72.390004) (width 0.3) (layer F.Cu) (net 6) (status 10))
 (via (at 76.2 72.390004) (size 1.6) (drill 1) (layers F.Cu B.Cu) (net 6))
 (segment (start 63.5 63.5) (end 63.5 72.390004) (width 0.3) (layer F.Cu) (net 6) (status 10))
 (via (at 63.5 72.390004) (size 1.6) (drill 1) (layers F.Cu B.Cu) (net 6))
 (segment (start 139.7 64.75) (end 139.7 63.5) (width 0.3) (layer B.Cu) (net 6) (status 20))
 (segment (start 50.8 63.5) (end 50.8 72.390004) (width 0.3) (layer F.Cu) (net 6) (status 10))
 (via (at 50.8 72.390004) (size 1.6) (drill 1) (layers F.Cu B.Cu) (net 6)))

